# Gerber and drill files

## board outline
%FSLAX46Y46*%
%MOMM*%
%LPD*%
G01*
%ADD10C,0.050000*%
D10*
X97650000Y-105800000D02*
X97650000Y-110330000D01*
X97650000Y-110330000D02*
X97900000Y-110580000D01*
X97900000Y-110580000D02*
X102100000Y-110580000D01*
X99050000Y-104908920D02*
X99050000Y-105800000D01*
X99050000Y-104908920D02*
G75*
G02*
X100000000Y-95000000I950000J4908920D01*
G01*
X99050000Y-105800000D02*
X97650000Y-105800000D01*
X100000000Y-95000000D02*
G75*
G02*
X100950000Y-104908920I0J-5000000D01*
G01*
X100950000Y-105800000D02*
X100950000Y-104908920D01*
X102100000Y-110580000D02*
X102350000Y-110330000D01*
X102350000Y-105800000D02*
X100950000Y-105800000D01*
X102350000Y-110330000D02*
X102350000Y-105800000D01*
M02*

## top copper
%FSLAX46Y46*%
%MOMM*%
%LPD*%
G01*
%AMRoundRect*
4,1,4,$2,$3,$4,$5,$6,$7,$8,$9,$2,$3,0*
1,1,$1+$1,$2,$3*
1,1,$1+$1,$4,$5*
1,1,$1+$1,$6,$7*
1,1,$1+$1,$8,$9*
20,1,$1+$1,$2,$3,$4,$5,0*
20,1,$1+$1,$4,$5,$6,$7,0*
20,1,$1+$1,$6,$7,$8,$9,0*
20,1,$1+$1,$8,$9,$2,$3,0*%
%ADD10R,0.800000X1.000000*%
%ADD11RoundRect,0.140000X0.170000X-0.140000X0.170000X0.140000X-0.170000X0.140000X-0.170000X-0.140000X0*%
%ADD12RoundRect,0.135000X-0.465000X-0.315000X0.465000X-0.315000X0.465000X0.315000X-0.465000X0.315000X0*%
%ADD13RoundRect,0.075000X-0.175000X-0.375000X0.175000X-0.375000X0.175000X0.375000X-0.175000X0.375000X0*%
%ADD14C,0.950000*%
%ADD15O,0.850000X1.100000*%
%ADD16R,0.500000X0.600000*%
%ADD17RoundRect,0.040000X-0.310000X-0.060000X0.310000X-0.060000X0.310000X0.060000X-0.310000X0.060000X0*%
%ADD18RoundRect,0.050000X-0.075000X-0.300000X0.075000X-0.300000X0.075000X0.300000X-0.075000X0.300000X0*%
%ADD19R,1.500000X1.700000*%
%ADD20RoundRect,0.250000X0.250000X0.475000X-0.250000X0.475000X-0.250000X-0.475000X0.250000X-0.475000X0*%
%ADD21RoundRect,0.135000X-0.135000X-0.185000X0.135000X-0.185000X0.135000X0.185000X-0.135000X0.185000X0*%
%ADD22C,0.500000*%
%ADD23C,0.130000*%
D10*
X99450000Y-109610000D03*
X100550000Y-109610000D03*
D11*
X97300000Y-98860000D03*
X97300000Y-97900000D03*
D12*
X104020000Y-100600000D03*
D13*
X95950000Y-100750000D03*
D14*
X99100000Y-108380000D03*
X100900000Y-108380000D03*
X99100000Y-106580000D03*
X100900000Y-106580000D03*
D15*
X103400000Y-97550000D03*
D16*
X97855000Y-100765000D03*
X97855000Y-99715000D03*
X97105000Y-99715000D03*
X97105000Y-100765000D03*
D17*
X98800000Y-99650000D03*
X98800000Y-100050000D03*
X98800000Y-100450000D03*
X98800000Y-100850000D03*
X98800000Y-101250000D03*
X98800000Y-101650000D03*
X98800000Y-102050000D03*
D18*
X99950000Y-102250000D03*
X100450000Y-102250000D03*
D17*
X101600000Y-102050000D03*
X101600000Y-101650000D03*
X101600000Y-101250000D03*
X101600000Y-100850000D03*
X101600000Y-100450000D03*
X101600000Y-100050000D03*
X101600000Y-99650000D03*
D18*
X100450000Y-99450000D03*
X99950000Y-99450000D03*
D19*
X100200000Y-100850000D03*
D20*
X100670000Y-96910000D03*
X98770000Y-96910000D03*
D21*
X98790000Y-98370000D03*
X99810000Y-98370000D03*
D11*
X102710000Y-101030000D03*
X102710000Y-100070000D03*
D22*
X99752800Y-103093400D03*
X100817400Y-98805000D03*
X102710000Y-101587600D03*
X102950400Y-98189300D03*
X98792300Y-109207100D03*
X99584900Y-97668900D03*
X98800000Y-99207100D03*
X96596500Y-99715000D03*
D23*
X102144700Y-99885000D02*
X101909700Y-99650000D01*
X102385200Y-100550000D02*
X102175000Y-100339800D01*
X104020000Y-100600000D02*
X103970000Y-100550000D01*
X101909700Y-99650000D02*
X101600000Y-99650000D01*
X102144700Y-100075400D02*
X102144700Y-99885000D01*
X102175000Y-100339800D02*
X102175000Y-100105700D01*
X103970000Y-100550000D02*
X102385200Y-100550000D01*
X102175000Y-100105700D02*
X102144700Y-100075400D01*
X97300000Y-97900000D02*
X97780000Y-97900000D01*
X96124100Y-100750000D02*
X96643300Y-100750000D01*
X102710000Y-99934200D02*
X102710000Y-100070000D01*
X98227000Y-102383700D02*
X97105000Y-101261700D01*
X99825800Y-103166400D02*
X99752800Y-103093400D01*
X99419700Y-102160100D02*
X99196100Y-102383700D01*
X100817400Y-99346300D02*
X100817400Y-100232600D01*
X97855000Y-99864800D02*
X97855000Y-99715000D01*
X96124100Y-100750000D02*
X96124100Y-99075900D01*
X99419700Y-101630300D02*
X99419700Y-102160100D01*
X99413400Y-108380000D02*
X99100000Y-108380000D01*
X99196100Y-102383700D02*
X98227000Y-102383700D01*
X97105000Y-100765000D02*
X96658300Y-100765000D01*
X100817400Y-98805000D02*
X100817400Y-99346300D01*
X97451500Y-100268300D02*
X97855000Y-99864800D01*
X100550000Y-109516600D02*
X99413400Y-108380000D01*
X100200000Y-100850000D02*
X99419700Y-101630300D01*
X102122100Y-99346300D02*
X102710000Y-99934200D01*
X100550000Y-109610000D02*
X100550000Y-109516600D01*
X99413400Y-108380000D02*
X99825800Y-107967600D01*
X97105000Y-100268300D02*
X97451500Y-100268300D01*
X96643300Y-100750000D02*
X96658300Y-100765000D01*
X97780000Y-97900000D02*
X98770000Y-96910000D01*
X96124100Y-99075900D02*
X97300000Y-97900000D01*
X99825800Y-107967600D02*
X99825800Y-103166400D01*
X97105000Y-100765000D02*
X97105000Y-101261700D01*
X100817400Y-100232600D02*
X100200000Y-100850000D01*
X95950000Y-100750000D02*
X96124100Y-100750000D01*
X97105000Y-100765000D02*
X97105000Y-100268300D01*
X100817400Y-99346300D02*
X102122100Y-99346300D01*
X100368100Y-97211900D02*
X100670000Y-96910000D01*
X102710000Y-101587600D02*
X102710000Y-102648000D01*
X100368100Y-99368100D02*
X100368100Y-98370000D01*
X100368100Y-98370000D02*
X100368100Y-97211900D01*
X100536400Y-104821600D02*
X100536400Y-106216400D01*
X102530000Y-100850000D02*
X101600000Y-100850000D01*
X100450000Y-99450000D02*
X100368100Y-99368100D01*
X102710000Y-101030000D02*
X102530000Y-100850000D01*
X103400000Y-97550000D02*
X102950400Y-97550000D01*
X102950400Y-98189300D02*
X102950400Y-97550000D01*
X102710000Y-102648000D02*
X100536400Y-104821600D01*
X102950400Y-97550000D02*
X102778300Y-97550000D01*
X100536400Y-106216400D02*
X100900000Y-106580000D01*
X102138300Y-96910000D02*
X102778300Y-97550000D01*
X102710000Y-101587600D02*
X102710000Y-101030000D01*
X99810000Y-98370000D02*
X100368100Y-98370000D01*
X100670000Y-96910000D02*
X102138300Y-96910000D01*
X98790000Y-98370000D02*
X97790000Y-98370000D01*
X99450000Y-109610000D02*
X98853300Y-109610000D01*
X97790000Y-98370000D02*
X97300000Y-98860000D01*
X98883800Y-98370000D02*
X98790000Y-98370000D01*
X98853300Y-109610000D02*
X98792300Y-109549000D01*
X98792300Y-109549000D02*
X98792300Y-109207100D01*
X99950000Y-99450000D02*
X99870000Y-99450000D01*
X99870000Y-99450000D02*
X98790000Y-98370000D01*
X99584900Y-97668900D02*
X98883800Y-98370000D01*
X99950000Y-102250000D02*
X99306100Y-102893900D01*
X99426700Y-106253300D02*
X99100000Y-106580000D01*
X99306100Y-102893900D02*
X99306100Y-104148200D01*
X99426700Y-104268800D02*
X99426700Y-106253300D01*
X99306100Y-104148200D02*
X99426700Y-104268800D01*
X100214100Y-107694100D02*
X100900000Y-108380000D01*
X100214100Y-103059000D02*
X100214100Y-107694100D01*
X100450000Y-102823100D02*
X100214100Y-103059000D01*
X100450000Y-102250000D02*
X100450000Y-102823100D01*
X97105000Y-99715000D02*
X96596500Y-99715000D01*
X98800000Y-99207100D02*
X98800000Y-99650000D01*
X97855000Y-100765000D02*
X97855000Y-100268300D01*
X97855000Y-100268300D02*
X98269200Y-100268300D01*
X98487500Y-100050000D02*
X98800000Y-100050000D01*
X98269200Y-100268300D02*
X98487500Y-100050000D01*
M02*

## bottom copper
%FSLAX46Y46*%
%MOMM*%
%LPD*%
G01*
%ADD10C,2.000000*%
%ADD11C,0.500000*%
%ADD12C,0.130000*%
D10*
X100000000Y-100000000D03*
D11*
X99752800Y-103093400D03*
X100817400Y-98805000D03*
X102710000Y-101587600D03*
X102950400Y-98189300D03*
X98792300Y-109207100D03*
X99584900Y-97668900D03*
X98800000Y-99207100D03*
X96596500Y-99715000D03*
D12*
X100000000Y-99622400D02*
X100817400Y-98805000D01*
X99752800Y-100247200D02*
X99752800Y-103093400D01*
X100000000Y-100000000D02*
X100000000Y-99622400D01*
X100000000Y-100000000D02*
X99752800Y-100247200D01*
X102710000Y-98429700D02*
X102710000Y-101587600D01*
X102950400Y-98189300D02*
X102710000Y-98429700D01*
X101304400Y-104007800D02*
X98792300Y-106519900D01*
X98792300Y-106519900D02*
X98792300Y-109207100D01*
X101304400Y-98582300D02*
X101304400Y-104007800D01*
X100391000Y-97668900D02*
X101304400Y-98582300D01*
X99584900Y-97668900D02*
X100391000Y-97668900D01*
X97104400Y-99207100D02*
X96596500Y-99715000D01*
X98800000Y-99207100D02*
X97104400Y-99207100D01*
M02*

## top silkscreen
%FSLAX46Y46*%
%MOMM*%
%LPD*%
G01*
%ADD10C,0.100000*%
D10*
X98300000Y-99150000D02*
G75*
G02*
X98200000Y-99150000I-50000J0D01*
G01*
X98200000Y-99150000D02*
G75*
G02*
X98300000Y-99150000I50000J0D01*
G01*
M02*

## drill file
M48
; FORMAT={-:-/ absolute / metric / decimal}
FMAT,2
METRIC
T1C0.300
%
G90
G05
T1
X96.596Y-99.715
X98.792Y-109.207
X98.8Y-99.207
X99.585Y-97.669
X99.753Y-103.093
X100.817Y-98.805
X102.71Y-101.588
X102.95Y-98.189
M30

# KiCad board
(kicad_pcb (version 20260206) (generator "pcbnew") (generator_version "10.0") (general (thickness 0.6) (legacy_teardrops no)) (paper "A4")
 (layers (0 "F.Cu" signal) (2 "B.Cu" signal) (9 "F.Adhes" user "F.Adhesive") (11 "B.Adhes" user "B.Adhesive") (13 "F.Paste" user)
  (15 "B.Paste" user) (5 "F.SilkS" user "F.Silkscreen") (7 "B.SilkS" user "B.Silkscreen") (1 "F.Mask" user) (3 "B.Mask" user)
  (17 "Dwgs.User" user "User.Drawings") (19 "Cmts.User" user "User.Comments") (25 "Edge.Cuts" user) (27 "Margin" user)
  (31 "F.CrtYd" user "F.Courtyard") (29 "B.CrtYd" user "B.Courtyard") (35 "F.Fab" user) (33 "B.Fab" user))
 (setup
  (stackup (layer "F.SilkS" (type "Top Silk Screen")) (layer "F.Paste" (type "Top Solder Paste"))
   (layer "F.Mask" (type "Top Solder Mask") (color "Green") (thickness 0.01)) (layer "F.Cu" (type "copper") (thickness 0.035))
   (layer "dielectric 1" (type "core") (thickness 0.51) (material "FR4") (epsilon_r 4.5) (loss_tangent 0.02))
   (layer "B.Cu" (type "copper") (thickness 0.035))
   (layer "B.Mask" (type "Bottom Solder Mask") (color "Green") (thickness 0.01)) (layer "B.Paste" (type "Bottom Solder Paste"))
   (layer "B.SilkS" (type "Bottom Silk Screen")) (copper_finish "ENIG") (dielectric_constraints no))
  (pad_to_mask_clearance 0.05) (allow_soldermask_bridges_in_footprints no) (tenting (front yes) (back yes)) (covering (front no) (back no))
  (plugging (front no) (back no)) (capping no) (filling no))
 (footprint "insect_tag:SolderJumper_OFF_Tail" (layer "F.Cu") (at 100 109.61 180)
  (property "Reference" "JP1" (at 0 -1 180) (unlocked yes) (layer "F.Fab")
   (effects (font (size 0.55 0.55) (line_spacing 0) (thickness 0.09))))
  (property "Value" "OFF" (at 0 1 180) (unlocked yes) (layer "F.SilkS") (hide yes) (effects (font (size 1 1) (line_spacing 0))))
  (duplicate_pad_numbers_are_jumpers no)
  (pad "1" smd rect (at 0.55 0 180) (size 0.8 1) (layers "F.Cu" "F.Mask") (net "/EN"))
  (pad "2" smd rect (at -0.55 0 180) (size 0.8 1) (layers "F.Cu" "F.Mask") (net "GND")))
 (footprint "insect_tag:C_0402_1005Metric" (layer "F.Cu") (at 97.3 98.38 90)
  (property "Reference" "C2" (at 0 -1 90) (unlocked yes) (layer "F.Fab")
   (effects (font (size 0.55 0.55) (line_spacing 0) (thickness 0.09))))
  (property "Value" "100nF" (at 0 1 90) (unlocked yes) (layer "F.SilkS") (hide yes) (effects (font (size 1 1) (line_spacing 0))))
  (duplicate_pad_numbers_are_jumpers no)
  (pad "1" smd roundrect (at -0.48 0 90) (size 0.56 0.62) (layers "F.Cu" "F.Mask" "F.Paste") (roundrect_rratio 0.25) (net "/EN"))
  (pad "2" smd roundrect (at 0.48 0 90) (size 0.56 0.62) (layers "F.Cu" "F.Mask" "F.Paste") (roundrect_rratio 0.25) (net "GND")))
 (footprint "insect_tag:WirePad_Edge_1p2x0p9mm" (layer "F.Cu") (at 104.02 100.6)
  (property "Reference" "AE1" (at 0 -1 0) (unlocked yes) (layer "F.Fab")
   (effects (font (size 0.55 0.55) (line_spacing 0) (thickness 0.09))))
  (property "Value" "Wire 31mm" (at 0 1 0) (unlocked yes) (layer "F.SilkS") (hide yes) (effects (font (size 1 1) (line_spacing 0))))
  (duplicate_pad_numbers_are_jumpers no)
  (pad "1" smd roundrect (at 0 0) (size 1.2 0.9) (layers "F.Cu" "F.Mask" "F.Paste") (roundrect_rratio 0.15) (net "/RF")))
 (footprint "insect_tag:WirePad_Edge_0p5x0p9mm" (layer "F.Cu") (at 95.95 100.75)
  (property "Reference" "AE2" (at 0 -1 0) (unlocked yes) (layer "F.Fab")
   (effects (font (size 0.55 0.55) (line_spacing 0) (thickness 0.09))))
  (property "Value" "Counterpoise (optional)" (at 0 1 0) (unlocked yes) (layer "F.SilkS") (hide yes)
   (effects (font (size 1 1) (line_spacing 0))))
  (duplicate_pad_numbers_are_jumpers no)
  (pad "1" smd roundrect (at 0 0) (size 0.5 0.9) (layers "F.Cu" "F.Mask" "F.Paste") (roundrect_rratio 0.15) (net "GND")))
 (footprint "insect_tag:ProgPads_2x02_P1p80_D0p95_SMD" (layer "F.Cu") (at 100 107.48)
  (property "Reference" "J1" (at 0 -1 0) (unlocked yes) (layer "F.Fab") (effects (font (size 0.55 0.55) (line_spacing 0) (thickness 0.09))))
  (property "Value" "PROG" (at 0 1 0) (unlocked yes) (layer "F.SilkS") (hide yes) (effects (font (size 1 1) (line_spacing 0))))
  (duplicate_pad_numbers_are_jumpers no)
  (pad "1" smd circle (at -0.9 0.9) (size 0.95 0.95) (layers "F.Cu" "F.Mask") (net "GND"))
  (pad "2" smd circle (at 0.9 0.9) (size 0.95 0.95) (layers "F.Cu" "F.Mask") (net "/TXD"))
  (pad "3" smd circle (at -0.9 -0.9) (size 0.95 0.95) (layers "F.Cu" "F.Mask") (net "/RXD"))
  (pad "4" smd circle (at 0.9 -0.9) (size 0.95 0.95) (layers "F.Cu" "F.Mask") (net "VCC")))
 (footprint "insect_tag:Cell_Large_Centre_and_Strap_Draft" (layer "F.Cu") (at 100 100)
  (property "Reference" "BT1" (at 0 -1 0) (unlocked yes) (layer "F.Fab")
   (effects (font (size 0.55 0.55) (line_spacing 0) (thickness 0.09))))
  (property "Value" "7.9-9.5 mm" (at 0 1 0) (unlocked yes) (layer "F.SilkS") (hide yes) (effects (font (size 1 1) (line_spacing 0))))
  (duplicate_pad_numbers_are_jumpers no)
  (pad "1" smd oval (at 3.4 -2.45) (size 0.85 1.1) (layers "F.Cu" "F.Mask") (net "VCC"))
  (pad "2" smd circle (at 0 0) (size 2 2) (layers "B.Cu" "B.Mask") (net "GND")))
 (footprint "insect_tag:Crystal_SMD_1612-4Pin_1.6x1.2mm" (layer "F.Cu") (at 97.48 100.24 90)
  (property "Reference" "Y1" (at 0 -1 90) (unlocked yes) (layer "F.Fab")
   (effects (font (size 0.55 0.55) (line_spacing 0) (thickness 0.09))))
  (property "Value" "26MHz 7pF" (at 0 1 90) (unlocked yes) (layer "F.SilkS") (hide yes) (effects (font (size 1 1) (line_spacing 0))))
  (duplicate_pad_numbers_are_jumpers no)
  (pad "1" smd rect (at -0.525 0.375 90) (size 0.6 0.5) (layers "F.Cu" "F.Mask" "F.Paste") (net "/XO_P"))
  (pad "2" smd rect (at 0.525 0.375 90) (size 0.6 0.5) (layers "F.Cu" "F.Mask" "F.Paste") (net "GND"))
  (pad "3" smd rect (at 0.525 -0.375 90) (size 0.6 0.5) (layers "F.Cu" "F.Mask" "F.Paste") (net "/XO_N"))
  (pad "4" smd rect (at -0.525 -0.375 90) (size 0.6 0.5) (layers "F.Cu" "F.Mask" "F.Paste") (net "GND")))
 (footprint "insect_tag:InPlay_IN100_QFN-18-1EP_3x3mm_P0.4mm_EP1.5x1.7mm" (layer "F.Cu") (at 100.2 100.85)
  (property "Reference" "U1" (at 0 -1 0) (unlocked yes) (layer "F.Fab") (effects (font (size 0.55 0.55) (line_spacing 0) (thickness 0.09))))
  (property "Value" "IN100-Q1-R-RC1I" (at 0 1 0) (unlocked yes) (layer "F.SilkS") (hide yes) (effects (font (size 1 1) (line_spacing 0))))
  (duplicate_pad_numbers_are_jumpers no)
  (fp_circle (center -1.95 -1.7) (end -1.9 -1.7) (stroke (width 0.1) (type solid)) (fill no) (layer "F.SilkS"))
  (pad "" smd rect (at 0 0) (size 0.24 1.5) (layers "F.Paste"))
  (pad "" smd rect (at 0 0) (size 1.3 0.34) (layers "F.Paste"))
  (pad "1" smd roundrect (at -1.4 -1.2) (size 0.7 0.2) (layers "F.Cu" "F.Mask" "F.Paste") (roundrect_rratio 0.2) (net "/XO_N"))
  (pad "2" smd roundrect (at -1.4 -0.8) (size 0.7 0.2) (layers "F.Cu" "F.Mask" "F.Paste") (roundrect_rratio 0.2) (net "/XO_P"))
  (pad "3" smd roundrect (at -1.4 -0.4) (size 0.7 0.2) (layers "F.Cu" "F.Mask" "F.Paste") (roundrect_rratio 0.2)
   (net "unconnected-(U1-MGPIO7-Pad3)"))
  (pad "4" smd roundrect (at -1.4 0) (size 0.7 0.2) (layers "F.Cu" "F.Mask" "F.Paste") (roundrect_rratio 0.2)
   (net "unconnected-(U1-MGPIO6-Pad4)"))
  (pad "5" smd roundrect (at -1.4 0.4) (size 0.7 0.2) (layers "F.Cu" "F.Mask" "F.Paste") (roundrect_rratio 0.2)
   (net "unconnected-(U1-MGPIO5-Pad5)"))
  (pad "6" smd roundrect (at -1.4 0.8) (size 0.7 0.2) (layers "F.Cu" "F.Mask" "F.Paste") (roundrect_rratio 0.2)
   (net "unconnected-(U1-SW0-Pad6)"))
  (pad "7" smd roundrect (at -1.4 1.2) (size 0.7 0.2) (layers "F.Cu" "F.Mask" "F.Paste") (roundrect_rratio 0.2)
   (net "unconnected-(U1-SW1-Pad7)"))
  (pad "8" smd roundrect (at -0.25 1.4) (size 0.25 0.7) (layers "F.Cu" "F.Mask" "F.Paste") (roundrect_rratio 0.2) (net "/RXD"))
  (pad "9" smd roundrect (at 0.25 1.4) (size 0.25 0.7) (layers "F.Cu" "F.Mask" "F.Paste") (roundrect_rratio 0.2) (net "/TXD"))
  (pad "10" smd roundrect (at 1.4 1.2) (size 0.7 0.2) (layers "F.Cu" "F.Mask" "F.Paste") (roundrect_rratio 0.2)
   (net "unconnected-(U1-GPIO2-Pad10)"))
  (pad "11" smd roundrect (at 1.4 0.8) (size 0.7 0.2) (layers "F.Cu" "F.Mask" "F.Paste") (roundrect_rratio 0.2)
   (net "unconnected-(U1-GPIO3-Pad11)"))
  (pad "12" smd roundrect (at 1.4 0.4) (size 0.7 0.2) (layers "F.Cu" "F.Mask" "F.Paste") (roundrect_rratio 0.2)
   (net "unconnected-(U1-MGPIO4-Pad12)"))
  (pad "13" smd roundrect (at 1.4 0) (size 0.7 0.2) (layers "F.Cu" "F.Mask" "F.Paste") (roundrect_rratio 0.2) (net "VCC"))
  (pad "14" smd roundrect (at 1.4 -0.4) (size 0.7 0.2) (layers "F.Cu" "F.Mask" "F.Paste") (roundrect_rratio 0.2)
   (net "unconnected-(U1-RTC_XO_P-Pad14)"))
  (pad "15" smd roundrect (at 1.4 -0.8) (size 0.7 0.2) (layers "F.Cu" "F.Mask" "F.Paste") (roundrect_rratio 0.2)
   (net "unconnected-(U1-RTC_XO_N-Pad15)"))
  (pad "16" smd roundrect (at 1.4 -1.2) (size 0.7 0.2) (layers "F.Cu" "F.Mask" "F.Paste") (roundrect_rratio 0.2) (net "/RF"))
  (pad "17" smd roundrect (at 0.25 -1.4) (size 0.25 0.7) (layers "F.Cu" "F.Mask" "F.Paste") (roundrect_rratio 0.2) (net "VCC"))
  (pad "18" smd roundrect (at -0.25 -1.4) (size 0.25 0.7) (layers "F.Cu" "F.Mask" "F.Paste") (roundrect_rratio 0.2) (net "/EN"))
  (pad "19" smd rect (at 0 0) (size 1.5 1.7) (layers "F.Cu" "F.Mask") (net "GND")))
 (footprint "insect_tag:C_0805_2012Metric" (layer "F.Cu") (at 99.72 96.91 180)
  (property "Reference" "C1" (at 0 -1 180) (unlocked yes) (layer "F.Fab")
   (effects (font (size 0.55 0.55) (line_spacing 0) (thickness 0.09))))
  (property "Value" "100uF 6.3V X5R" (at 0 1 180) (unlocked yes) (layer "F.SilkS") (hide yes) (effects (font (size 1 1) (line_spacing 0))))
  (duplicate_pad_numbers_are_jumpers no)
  (pad "1" smd roundrect (at -0.95 0 180) (size 1 1.45) (layers "F.Cu" "F.Mask" "F.Paste") (roundrect_rratio 0.25) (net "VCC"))
  (pad "2" smd roundrect (at 0.95 0 180) (size 1 1.45) (layers "F.Cu" "F.Mask" "F.Paste") (roundrect_rratio 0.25) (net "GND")))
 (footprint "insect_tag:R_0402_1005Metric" (layer "F.Cu") (at 99.3 98.37)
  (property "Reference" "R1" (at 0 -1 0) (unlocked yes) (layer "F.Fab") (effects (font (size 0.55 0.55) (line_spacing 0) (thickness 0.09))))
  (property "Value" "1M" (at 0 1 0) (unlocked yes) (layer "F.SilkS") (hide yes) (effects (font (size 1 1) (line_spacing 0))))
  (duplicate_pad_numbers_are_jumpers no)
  (pad "1" smd roundrect (at -0.51 0) (size 0.54 0.64) (layers "F.Cu" "F.Mask" "F.Paste") (roundrect_rratio 0.25) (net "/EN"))
  (pad "2" smd roundrect (at 0.51 0) (size 0.54 0.64) (layers "F.Cu" "F.Mask" "F.Paste") (roundrect_rratio 0.25) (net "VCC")))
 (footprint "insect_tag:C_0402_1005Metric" (layer "F.Cu") (at 102.71 100.55 90)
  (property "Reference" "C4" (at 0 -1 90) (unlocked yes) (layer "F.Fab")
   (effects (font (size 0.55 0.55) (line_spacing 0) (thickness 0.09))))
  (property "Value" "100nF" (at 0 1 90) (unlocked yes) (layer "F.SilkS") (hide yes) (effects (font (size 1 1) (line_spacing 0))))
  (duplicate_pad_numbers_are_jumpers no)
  (pad "1" smd roundrect (at -0.48 0 90) (size 0.56 0.62) (layers "F.Cu" "F.Mask" "F.Paste") (roundrect_rratio 0.25) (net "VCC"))
  (pad "2" smd roundrect (at 0.48 0 90) (size 0.56 0.62) (layers "F.Cu" "F.Mask" "F.Paste") (roundrect_rratio 0.25) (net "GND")))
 (gr_line (start 97.65 105.8) (end 97.65 110.33) (stroke (width 0.05) (type default)) (layer "Edge.Cuts"))
 (gr_line (start 97.65 110.33) (end 97.9 110.58) (stroke (width 0.05) (type default)) (layer "Edge.Cuts"))
 (gr_line (start 97.9 110.58) (end 102.1 110.58) (stroke (width 0.05) (type default)) (layer "Edge.Cuts"))
 (gr_line (start 99.05 104.90892) (end 99.05 105.8) (stroke (width 0.05) (type default)) (layer "Edge.Cuts"))
 (gr_arc (start 99.05 104.90892) (mid 95.022822 99.522822) (end 100 95) (stroke (width 0.05) (type default)) (layer "Edge.Cuts"))
 (gr_line (start 99.05 105.8) (end 97.65 105.8) (stroke (width 0.05) (type default)) (layer "Edge.Cuts"))
 (gr_arc (start 100 95) (mid 104.977178 99.522822) (end 100.95 104.90892) (stroke (width 0.05) (type default)) (layer "Edge.Cuts"))
 (gr_line (start 100.95 105.8) (end 100.95 104.90892) (stroke (width 0.05) (type default)) (layer "Edge.Cuts"))
 (gr_line (start 102.1 110.58) (end 102.35 110.33) (stroke (width 0.05) (type default)) (layer "Edge.Cuts"))
 (gr_line (start 102.35 105.8) (end 100.95 105.8) (stroke (width 0.05) (type default)) (layer "Edge.Cuts"))
 (gr_line (start 102.35 110.33) (end 102.35 105.8) (stroke (width 0.05) (type default)) (layer "Edge.Cuts"))
 (segment (start 102.1447 99.885) (end 101.9097 99.65) (width 0.13) (layer "F.Cu") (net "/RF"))
 (segment (start 102.3852 100.55) (end 102.175 100.3398) (width 0.13) (layer "F.Cu") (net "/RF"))
 (segment (start 104.02 100.6) (end 103.97 100.55) (width 0.13) (layer "F.Cu") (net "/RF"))
 (segment (start 101.9097 99.65) (end 101.6 99.65) (width 0.13) (layer "F.Cu") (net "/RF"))
 (segment (start 102.1447 100.0754) (end 102.1447 99.885) (width 0.13) (layer "F.Cu") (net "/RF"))
 (segment (start 102.175 100.3398) (end 102.175 100.1057) (width 0.13) (layer "F.Cu") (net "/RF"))
 (segment (start 103.97 100.55) (end 102.3852 100.55) (width 0.13) (layer "F.Cu") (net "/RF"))
 (segment (start 102.175 100.1057) (end 102.1447 100.0754) (width 0.13) (layer "F.Cu") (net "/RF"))
 (segment (start 97.3 97.9) (end 97.78 97.9) (width 0.13) (layer "F.Cu") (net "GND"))
 (segment (start 96.1241 100.75) (end 96.6433 100.75) (width 0.13) (layer "F.Cu") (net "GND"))
 (segment (start 102.71 99.9342) (end 102.71 100.07) (width 0.13) (layer "F.Cu") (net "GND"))
 (segment (start 98.227 102.3837) (end 97.105 101.2617) (width 0.13) (layer "F.Cu") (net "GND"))
 (segment (start 99.8258 103.1664) (end 99.7528 103.0934) (width 0.13) (layer "F.Cu") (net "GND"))
 (segment (start 99.4197 102.1601) (end 99.1961 102.3837) (width 0.13) (layer "F.Cu") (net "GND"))
 (segment (start 100.8174 99.3463) (end 100.8174 100.2326) (width 0.13) (layer "F.Cu") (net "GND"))
 (segment (start 97.855 99.8648) (end 97.855 99.715) (width 0.13) (layer "F.Cu") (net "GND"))
 (segment (start 96.1241 100.75) (end 96.1241 99.0759) (width 0.13) (layer "F.Cu") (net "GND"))
 (segment (start 99.4197 101.6303) (end 99.4197 102.1601) (width 0.13) (layer "F.Cu") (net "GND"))
 (segment (start 99.4134 108.38) (end 99.1 108.38) (width 0.13) (layer "F.Cu") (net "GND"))
 (segment (start 99.1961 102.3837) (end 98.227 102.3837) (width 0.13) (layer "F.Cu") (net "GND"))
 (segment (start 97.105 100.765) (end 96.6583 100.765) (width 0.13) (layer "F.Cu") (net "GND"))
 (segment (start 100.8174 98.805) (end 100.8174 99.3463) (width 0.13) (layer "F.Cu") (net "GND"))
 (segment (start 97.4515 100.2683) (end 97.855 99.8648) (width 0.13) (layer "F.Cu") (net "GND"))
 (segment (start 100.55 109.5166) (end 99.4134 108.38) (width 0.13) (layer "F.Cu") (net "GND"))
 (segment (start 100.2 100.85) (end 99.4197 101.6303) (width 0.13) (layer "F.Cu") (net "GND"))
 (segment (start 102.1221 99.3463) (end 102.71 99.9342) (width 0.13) (layer "F.Cu") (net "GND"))
 (segment (start 100.55 109.61) (end 100.55 109.5166) (width 0.13) (layer "F.Cu") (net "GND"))
 (segment (start 99.4134 108.38) (end 99.8258 107.9676) (width 0.13) (layer "F.Cu") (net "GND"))
 (segment (start 97.105 100.2683) (end 97.4515 100.2683) (width 0.13) (layer "F.Cu") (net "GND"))
 (segment (start 96.6433 100.75) (end 96.6583 100.765) (width 0.13) (layer "F.Cu") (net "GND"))
 (segment (start 97.78 97.9) (end 98.77 96.91) (width 0.13) (layer "F.Cu") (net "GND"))
 (segment (start 96.1241 99.0759) (end 97.3 97.9) (width 0.13) (layer "F.Cu") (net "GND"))
 (segment (start 99.8258 107.9676) (end 99.8258 103.1664) (width 0.13) (layer "F.Cu") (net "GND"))
 (segment (start 97.105 100.765) (end 97.105 101.2617) (width 0.13) (layer "F.Cu") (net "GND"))
 (segment (start 100.8174 100.2326) (end 100.2 100.85) (width 0.13) (layer "F.Cu") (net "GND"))
 (segment (start 95.95 100.75) (end 96.1241 100.75) (width 0.13) (layer "F.Cu") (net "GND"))
 (segment (start 97.105 100.765) (end 97.105 100.2683) (width 0.13) (layer "F.Cu") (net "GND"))
 (segment (start 100.8174 99.3463) (end 102.1221 99.3463) (width 0.13) (layer "F.Cu") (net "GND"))
 (via (at 99.7528 103.0934) (size 0.5) (drill 0.3) (layers "F.Cu" "B.Cu") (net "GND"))
 (via (at 100.8174 98.805) (size 0.5) (drill 0.3) (layers "F.Cu" "B.Cu") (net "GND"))
 (segment (start 100 99.6224) (end 100.8174 98.805) (width 0.13) (layer "B.Cu") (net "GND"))
 (segment (start 99.7528 100.2472) (end 99.7528 103.0934) (width 0.13) (layer "B.Cu") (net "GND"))
 (segment (start 100 100) (end 100 99.6224) (width 0.13) (layer "B.Cu") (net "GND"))
 (segment (start 100 100) (end 99.7528 100.2472) (width 0.13) (layer "B.Cu") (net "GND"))
 (segment (start 100.3681 97.2119) (end 100.67 96.91) (width 0.13) (layer "F.Cu") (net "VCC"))
 (segment (start 102.71 101.5876) (end 102.71 102.648) (width 0.13) (layer "F.Cu") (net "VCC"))
 (segment (start 100.3681 99.3681) (end 100.3681 98.37) (width 0.13) (layer "F.Cu") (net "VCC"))
 (segment (start 100.3681 98.37) (end 100.3681 97.2119) (width 0.13) (layer "F.Cu") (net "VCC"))
 (segment (start 100.5364 104.8216) (end 100.5364 106.2164) (width 0.13) (layer "F.Cu") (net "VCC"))
 (segment (start 102.53 100.85) (end 101.6 100.85) (width 0.13) (layer "F.Cu") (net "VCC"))
 (segment (start 100.45 99.45) (end 100.3681 99.3681) (width 0.13) (layer "F.Cu") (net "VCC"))
 (segment (start 102.71 101.03) (end 102.53 100.85) (width 0.13) (layer "F.Cu") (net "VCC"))
 (segment (start 103.4 97.55) (end 102.9504 97.55) (width 0.13) (layer "F.Cu") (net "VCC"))
 (segment (start 102.9504 98.1893) (end 102.9504 97.55) (width 0.13) (layer "F.Cu") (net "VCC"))
 (segment (start 102.71 102.648) (end 100.5364 104.8216) (width 0.13) (layer "F.Cu") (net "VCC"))
 (segment (start 102.9504 97.55) (end 102.7783 97.55) (width 0.13) (layer "F.Cu") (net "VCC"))
 (segment (start 100.5364 106.2164) (end 100.9 106.58) (width 0.13) (layer "F.Cu") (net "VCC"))
 (segment (start 102.1383 96.91) (end 102.7783 97.55) (width 0.13) (layer "F.Cu") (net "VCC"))
 (segment (start 102.71 101.5876) (end 102.71 101.03) (width 0.13) (layer "F.Cu") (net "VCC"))
 (segment (start 99.81 98.37) (end 100.3681 98.37) (width 0.13) (layer "F.Cu") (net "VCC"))
 (segment (start 100.67 96.91) (end 102.1383 96.91) (width 0.13) (layer "F.Cu") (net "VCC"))
 (via (at 102.71 101.5876) (size 0.5) (drill 0.3) (layers "F.Cu" "B.Cu") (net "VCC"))
 (via (at 102.9504 98.1893) (size 0.5) (drill 0.3) (layers "F.Cu" "B.Cu") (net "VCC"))
 (segment (start 102.71 98.4297) (end 102.71 101.5876) (width 0.13) (layer "B.Cu") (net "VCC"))
 (segment (start 102.9504 98.1893) (end 102.71 98.4297) (width 0.13) (layer "B.Cu") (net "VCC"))
 (segment (start 98.79 98.37) (end 97.79 98.37) (width 0.13) (layer "F.Cu") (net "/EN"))
 (segment (start 99.45 109.61) (end 98.8533 109.61) (width 0.13) (layer "F.Cu") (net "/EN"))
 (segment (start 97.79 98.37) (end 97.3 98.86) (width 0.13) (layer "F.Cu") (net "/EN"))
 (segment (start 98.8838 98.37) (end 98.79 98.37) (width 0.13) (layer "F.Cu") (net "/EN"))
 (segment (start 98.8533 109.61) (end 98.7923 109.549) (width 0.13) (layer "F.Cu") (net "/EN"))
 (segment (start 98.7923 109.549) (end 98.7923 109.2071) (width 0.13) (layer "F.Cu") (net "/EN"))
 (segment (start 99.95 99.45) (end 99.87 99.45) (width 0.13) (layer "F.Cu") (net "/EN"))
 (segment (start 99.87 99.45) (end 98.79 98.37) (width 0.13) (layer "F.Cu") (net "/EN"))
 (segment (start 99.5849 97.6689) (end 98.8838 98.37) (width 0.13) (layer "F.Cu") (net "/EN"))
 (via (at 98.7923 109.2071) (size 0.5) (drill 0.3) (layers "F.Cu" "B.Cu") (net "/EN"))
 (via (at 99.5849 97.6689) (size 0.5) (drill 0.3) (layers "F.Cu" "B.Cu") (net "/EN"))
 (segment (start 101.3044 104.0078) (end 98.7923 106.5199) (width 0.13) (layer "B.Cu") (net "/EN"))
 (segment (start 98.7923 106.5199) (end 98.7923 109.2071) (width 0.13) (layer "B.Cu") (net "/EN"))
 (segment (start 101.3044 98.5823) (end 101.3044 104.0078) (width 0.13) (layer "B.Cu") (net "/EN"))
 (segment (start 100.391 97.6689) (end 101.3044 98.5823) (width 0.13) (layer "B.Cu") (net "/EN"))
 (segment (start 99.5849 97.6689) (end 100.391 97.6689) (width 0.13) (layer "B.Cu") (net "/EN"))
 (segment (start 99.95 102.25) (end 99.3061 102.8939) (width 0.13) (layer "F.Cu") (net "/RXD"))
 (segment (start 99.4267 106.2533) (end 99.1 106.58) (width 0.13) (layer "F.Cu") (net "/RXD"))
 (segment (start 99.3061 102.8939) (end 99.3061 104.1482) (width 0.13) (layer "F.Cu") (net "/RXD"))
 (segment (start 99.4267 104.2688) (end 99.4267 106.2533) (width 0.13) (layer "F.Cu") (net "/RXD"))
 (segment (start 99.3061 104.1482) (end 99.4267 104.2688) (width 0.13) (layer "F.Cu") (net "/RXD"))
 (segment (start 100.2141 107.6941) (end 100.9 108.38) (width 0.13) (layer "F.Cu") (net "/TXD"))
 (segment (start 100.2141 103.059) (end 100.2141 107.6941) (width 0.13) (layer "F.Cu") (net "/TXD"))
 (segment (start 100.45 102.8231) (end 100.2141 103.059) (width 0.13) (layer "F.Cu") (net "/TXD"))
 (segment (start 100.45 102.25) (end 100.45 102.8231) (width 0.13) (layer "F.Cu") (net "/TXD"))
 (segment (start 97.105 99.715) (end 96.5965 99.715) (width 0.13) (layer "F.Cu") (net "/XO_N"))
 (segment (start 98.8 99.2071) (end 98.8 99.65) (width 0.13) (layer "F.Cu") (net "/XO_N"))
 (via (at 98.8 99.2071) (size 0.5) (drill 0.3) (layers "F.Cu" "B.Cu") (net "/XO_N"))
 (via (at 96.5965 99.715) (size 0.5) (drill 0.3) (layers "F.Cu" "B.Cu") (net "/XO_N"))
 (segment (start 97.1044 99.2071) (end 96.5965 99.715) (width 0.13) (layer "B.Cu") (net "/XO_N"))
 (segment (start 98.8 99.2071) (end 97.1044 99.2071) (width 0.13) (layer "B.Cu") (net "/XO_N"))
 (segment (start 97.855 100.765) (end 97.855 100.2683) (width 0.13) (layer "F.Cu") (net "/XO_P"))
 (segment (start 97.855 100.2683) (end 98.2692 100.2683) (width 0.13) (layer "F.Cu") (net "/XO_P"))
 (segment (start 98.4875 100.05) (end 98.8 100.05) (width 0.13) (layer "F.Cu") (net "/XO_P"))
 (segment (start 98.2692 100.2683) (end 98.4875 100.05) (width 0.13) (layer "F.Cu") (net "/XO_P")))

